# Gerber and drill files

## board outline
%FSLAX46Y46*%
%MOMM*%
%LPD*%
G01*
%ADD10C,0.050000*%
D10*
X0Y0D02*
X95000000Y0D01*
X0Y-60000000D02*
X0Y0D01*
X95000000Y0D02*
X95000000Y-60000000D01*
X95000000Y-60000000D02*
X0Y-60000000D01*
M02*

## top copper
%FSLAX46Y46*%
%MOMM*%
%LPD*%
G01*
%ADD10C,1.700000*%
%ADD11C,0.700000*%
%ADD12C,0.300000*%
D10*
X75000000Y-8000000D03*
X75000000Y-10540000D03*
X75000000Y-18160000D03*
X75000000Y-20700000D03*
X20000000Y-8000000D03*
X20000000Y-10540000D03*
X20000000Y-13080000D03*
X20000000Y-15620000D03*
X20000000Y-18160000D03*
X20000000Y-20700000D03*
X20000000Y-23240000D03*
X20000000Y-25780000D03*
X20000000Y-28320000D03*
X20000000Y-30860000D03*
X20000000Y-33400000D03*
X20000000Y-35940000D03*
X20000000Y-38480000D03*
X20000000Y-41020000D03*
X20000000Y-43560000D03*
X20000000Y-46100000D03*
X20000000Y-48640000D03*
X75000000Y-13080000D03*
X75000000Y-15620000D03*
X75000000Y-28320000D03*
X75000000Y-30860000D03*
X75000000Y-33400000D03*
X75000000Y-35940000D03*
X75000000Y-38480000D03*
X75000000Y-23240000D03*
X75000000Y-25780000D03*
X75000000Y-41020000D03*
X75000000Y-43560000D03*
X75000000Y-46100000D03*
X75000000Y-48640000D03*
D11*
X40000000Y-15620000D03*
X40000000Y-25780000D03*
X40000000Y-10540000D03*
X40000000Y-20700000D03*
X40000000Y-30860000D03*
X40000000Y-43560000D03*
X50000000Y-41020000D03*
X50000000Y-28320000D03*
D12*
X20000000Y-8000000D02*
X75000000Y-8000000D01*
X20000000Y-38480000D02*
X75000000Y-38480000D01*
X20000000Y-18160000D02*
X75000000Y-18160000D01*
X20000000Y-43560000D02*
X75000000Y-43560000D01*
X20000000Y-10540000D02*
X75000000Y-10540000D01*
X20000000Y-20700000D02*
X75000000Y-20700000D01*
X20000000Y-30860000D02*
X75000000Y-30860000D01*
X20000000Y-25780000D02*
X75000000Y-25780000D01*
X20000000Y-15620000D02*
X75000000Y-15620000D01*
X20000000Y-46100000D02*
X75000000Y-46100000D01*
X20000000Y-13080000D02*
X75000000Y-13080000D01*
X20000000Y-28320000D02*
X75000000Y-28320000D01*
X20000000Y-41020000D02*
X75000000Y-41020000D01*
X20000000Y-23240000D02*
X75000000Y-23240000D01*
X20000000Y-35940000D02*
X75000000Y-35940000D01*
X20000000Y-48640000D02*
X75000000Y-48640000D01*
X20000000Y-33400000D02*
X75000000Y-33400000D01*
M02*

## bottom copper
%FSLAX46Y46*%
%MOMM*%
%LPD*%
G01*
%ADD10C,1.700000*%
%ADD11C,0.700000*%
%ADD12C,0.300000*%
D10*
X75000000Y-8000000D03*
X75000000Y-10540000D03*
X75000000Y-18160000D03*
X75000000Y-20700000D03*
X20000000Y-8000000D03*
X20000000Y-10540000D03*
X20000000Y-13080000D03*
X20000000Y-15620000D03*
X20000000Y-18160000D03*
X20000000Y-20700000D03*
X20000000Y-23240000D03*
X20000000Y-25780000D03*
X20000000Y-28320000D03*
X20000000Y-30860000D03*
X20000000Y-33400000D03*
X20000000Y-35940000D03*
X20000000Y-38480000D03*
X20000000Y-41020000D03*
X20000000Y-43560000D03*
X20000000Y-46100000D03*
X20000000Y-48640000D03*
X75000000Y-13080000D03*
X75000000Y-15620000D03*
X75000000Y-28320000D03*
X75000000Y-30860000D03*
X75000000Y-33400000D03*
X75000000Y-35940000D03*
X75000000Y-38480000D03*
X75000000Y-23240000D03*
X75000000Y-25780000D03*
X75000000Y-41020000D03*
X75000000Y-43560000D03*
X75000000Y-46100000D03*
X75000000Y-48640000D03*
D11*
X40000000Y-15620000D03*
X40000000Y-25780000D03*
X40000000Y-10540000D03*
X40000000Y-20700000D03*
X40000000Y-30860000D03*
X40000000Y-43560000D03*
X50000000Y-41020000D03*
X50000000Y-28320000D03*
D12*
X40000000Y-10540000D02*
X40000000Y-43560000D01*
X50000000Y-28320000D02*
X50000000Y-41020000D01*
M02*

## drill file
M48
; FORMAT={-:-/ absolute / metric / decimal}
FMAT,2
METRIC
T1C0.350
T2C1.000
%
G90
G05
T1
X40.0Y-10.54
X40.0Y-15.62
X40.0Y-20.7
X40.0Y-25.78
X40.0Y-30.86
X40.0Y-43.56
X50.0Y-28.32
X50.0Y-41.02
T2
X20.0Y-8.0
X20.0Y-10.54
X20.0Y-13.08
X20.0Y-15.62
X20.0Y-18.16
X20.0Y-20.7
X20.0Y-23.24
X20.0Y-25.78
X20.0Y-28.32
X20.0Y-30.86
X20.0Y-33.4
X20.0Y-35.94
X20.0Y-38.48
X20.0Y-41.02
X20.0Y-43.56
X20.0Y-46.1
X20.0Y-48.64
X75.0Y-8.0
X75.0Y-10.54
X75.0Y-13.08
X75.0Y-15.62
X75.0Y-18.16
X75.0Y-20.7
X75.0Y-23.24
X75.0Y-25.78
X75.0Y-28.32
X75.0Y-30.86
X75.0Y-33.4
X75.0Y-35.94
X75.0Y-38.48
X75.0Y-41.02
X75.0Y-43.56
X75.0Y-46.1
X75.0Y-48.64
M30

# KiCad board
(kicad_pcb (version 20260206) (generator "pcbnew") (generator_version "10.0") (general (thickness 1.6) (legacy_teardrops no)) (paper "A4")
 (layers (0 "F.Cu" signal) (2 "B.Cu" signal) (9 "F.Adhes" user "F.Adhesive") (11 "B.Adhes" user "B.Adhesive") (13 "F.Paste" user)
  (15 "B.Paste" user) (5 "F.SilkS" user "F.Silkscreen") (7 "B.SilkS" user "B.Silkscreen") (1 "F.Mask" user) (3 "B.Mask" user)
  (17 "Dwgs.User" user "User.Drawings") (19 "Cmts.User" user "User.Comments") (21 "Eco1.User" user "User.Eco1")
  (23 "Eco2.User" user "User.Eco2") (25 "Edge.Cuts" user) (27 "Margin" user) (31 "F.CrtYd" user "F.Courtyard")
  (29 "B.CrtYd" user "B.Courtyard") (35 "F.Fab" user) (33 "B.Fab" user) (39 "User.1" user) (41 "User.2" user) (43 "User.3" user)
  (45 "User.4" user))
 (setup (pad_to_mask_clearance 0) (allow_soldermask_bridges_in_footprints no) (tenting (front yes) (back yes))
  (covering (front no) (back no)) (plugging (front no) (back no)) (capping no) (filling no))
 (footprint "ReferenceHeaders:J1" (layer "F.Cu") (at 75 8)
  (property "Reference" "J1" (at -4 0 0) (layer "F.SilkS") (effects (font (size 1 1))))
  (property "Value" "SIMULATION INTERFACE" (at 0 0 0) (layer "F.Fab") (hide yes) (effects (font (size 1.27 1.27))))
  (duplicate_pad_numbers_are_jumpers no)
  (pad "1" thru_hole circle (at 0 0) (size 1.7 1.7) (drill 1) (layers "*.Cu" "*.Mask") (remove_unused_layers no) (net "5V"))
  (pad "2" thru_hole circle (at 0 2.54) (size 1.7 1.7) (drill 1) (layers "*.Cu" "*.Mask") (remove_unused_layers no) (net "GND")))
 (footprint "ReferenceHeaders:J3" (layer "F.Cu") (at 75 18.16)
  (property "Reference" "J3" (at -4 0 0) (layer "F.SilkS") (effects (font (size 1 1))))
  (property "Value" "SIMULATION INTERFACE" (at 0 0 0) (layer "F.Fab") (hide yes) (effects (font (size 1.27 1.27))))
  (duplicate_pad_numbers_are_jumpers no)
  (pad "1" thru_hole circle (at 0 0) (size 1.7 1.7) (drill 1) (layers "*.Cu" "*.Mask") (remove_unused_layers no) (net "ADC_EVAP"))
  (pad "2" thru_hole circle (at 0 2.54) (size 1.7 1.7) (drill 1) (layers "*.Cu" "*.Mask") (remove_unused_layers no) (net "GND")))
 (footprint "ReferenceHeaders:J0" (layer "F.Cu") (at 20 8)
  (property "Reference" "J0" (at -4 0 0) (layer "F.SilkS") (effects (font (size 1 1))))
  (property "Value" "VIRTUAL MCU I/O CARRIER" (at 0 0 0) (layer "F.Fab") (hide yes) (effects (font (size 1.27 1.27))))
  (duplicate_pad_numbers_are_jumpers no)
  (pad "1" thru_hole circle (at 0 0) (size 1.7 1.7) (drill 1) (layers "*.Cu" "*.Mask") (remove_unused_layers no) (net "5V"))
  (pad "2" thru_hole circle (at 0 2.54) (size 1.7 1.7) (drill 1) (layers "*.Cu" "*.Mask") (remove_unused_layers no) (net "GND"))
  (pad "3" thru_hole circle (at 0 5.08) (size 1.7 1.7) (drill 1) (layers "*.Cu" "*.Mask") (remove_unused_layers no) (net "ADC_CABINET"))
  (pad "4" thru_hole circle (at 0 7.62) (size 1.7 1.7) (drill 1) (layers "*.Cu" "*.Mask") (remove_unused_layers no) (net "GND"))
  (pad "5" thru_hole circle (at 0 10.16) (size 1.7 1.7) (drill 1) (layers "*.Cu" "*.Mask") (remove_unused_layers no) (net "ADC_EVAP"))
  (pad "6" thru_hole circle (at 0 12.7) (size 1.7 1.7) (drill 1) (layers "*.Cu" "*.Mask") (remove_unused_layers no) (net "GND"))
  (pad "7" thru_hole circle (at 0 15.24) (size 1.7 1.7) (drill 1) (layers "*.Cu" "*.Mask") (remove_unused_layers no)
   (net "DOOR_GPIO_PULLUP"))
  (pad "8" thru_hole circle (at 0 17.78) (size 1.7 1.7) (drill 1) (layers "*.Cu" "*.Mask") (remove_unused_layers no) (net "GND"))
  (pad "9" thru_hole circle (at 0 20.32) (size 1.7 1.7) (drill 1) (layers "*.Cu" "*.Mask") (remove_unused_layers no) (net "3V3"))
  (pad "10" thru_hole circle (at 0 22.86) (size 1.7 1.7) (drill 1) (layers "*.Cu" "*.Mask") (remove_unused_layers no) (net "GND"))
  (pad "11" thru_hole circle (at 0 25.4) (size 1.7 1.7) (drill 1) (layers "*.Cu" "*.Mask") (remove_unused_layers no) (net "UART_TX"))
  (pad "12" thru_hole circle (at 0 27.94) (size 1.7 1.7) (drill 1) (layers "*.Cu" "*.Mask") (remove_unused_layers no) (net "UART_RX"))
  (pad "13" thru_hole circle (at 0 30.48) (size 1.7 1.7) (drill 1) (layers "*.Cu" "*.Mask") (remove_unused_layers no) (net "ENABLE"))
  (pad "14" thru_hole circle (at 0 33.02) (size 1.7 1.7) (drill 1) (layers "*.Cu" "*.Mask") (remove_unused_layers no) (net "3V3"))
  (pad "15" thru_hole circle (at 0 35.56) (size 1.7 1.7) (drill 1) (layers "*.Cu" "*.Mask") (remove_unused_layers no) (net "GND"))
  (pad "16" thru_hole circle (at 0 38.1) (size 1.7 1.7) (drill 1) (layers "*.Cu" "*.Mask") (remove_unused_layers no) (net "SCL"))
  (pad "17" thru_hole circle (at 0 40.64) (size 1.7 1.7) (drill 1) (layers "*.Cu" "*.Mask") (remove_unused_layers no) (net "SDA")))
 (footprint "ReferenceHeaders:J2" (layer "F.Cu") (at 75 13.08)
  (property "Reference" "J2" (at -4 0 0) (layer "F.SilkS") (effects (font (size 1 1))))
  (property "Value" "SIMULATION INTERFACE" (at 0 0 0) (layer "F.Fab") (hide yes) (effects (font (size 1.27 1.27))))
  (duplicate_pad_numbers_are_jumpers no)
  (pad "1" thru_hole circle (at 0 0) (size 1.7 1.7) (drill 1) (layers "*.Cu" "*.Mask") (remove_unused_layers no) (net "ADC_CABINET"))
  (pad "2" thru_hole circle (at 0 2.54) (size 1.7 1.7) (drill 1) (layers "*.Cu" "*.Mask") (remove_unused_layers no) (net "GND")))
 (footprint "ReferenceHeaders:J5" (layer "F.Cu") (at 75 28.32)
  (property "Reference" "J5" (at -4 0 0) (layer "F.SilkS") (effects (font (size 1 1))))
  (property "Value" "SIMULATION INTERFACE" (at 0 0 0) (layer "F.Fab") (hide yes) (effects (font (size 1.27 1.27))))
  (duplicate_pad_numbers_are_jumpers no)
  (pad "1" thru_hole circle (at 0 0) (size 1.7 1.7) (drill 1) (layers "*.Cu" "*.Mask") (remove_unused_layers no) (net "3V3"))
  (pad "2" thru_hole circle (at 0 2.54) (size 1.7 1.7) (drill 1) (layers "*.Cu" "*.Mask") (remove_unused_layers no) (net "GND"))
  (pad "3" thru_hole circle (at 0 5.08) (size 1.7 1.7) (drill 1) (layers "*.Cu" "*.Mask") (remove_unused_layers no) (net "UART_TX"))
  (pad "4" thru_hole circle (at 0 7.62) (size 1.7 1.7) (drill 1) (layers "*.Cu" "*.Mask") (remove_unused_layers no) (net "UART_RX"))
  (pad "5" thru_hole circle (at 0 10.16) (size 1.7 1.7) (drill 1) (layers "*.Cu" "*.Mask") (remove_unused_layers no) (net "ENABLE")))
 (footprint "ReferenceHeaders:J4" (layer "F.Cu") (at 75 23.24)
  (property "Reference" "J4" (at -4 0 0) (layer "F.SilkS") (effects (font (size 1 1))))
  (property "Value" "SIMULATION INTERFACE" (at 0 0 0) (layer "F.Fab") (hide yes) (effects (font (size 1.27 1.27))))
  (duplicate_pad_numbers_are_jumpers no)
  (pad "1" thru_hole circle (at 0 0) (size 1.7 1.7) (drill 1) (layers "*.Cu" "*.Mask") (remove_unused_layers no) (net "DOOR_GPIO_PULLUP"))
  (pad "2" thru_hole circle (at 0 2.54) (size 1.7 1.7) (drill 1) (layers "*.Cu" "*.Mask") (remove_unused_layers no) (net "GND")))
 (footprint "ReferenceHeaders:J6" (layer "F.Cu") (at 75 41.02)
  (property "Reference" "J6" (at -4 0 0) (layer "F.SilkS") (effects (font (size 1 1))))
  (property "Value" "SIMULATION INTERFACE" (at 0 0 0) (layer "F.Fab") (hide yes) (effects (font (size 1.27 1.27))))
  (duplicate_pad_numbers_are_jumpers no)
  (pad "1" thru_hole circle (at 0 0) (size 1.7 1.7) (drill 1) (layers "*.Cu" "*.Mask") (remove_unused_layers no) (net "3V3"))
  (pad "2" thru_hole circle (at 0 2.54) (size 1.7 1.7) (drill 1) (layers "*.Cu" "*.Mask") (remove_unused_layers no) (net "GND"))
  (pad "3" thru_hole circle (at 0 5.08) (size 1.7 1.7) (drill 1) (layers "*.Cu" "*.Mask") (remove_unused_layers no) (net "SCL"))
  (pad "4" thru_hole circle (at 0 7.62) (size 1.7 1.7) (drill 1) (layers "*.Cu" "*.Mask") (remove_unused_layers no) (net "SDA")))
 (gr_line (start 0 0) (end 95 0) (stroke (width 0.05) (type default)) (layer "Edge.Cuts"))
 (gr_line (start 0 60) (end 0 0) (stroke (width 0.05) (type default)) (layer "Edge.Cuts"))
 (gr_line (start 95 0) (end 95 60) (stroke (width 0.05) (type default)) (layer "Edge.Cuts"))
 (gr_line (start 95 60) (end 0 60) (stroke (width 0.05) (type default)) (layer "Edge.Cuts"))
 (segment (start 20 8) (end 75 8) (width 0.3) (layer "F.Cu") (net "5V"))
 (segment (start 20 38.48) (end 75 38.48) (width 0.3) (layer "F.Cu") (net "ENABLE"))
 (segment (start 20 18.16) (end 75 18.16) (width 0.3) (layer "F.Cu") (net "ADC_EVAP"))
 (segment (start 20 43.56) (end 75 43.56) (width 0.3) (layer "F.Cu") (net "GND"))
 (segment (start 20 10.54) (end 75 10.54) (width 0.3) (layer "F.Cu") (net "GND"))
 (segment (start 20 20.7) (end 75 20.7) (width 0.3) (layer "F.Cu") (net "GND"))
 (segment (start 20 30.86) (end 75 30.86) (width 0.3) (layer "F.Cu") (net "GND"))
 (segment (start 20 25.78) (end 75 25.78) (width 0.3) (layer "F.Cu") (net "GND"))
 (segment (start 20 15.62) (end 75 15.62) (width 0.3) (layer "F.Cu") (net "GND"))
 (via (at 40 15.62) (size 0.7) (drill 0.35) (layers "F.Cu" "B.Cu") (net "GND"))
 (via (at 40 25.78) (size 0.7) (drill 0.35) (layers "F.Cu" "B.Cu") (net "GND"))
 (via (at 40 10.54) (size 0.7) (drill 0.35) (layers "F.Cu" "B.Cu") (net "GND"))
 (via (at 40 20.7) (size 0.7) (drill 0.35) (layers "F.Cu" "B.Cu") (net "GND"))
 (via (at 40 30.86) (size 0.7) (drill 0.35) (layers "F.Cu" "B.Cu") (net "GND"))
 (via (at 40 43.56) (size 0.7) (drill 0.35) (layers "F.Cu" "B.Cu") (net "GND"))
 (segment (start 40 10.54) (end 40 43.56) (width 0.3) (layer "B.Cu") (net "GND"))
 (segment (start 20 46.1) (end 75 46.1) (width 0.3) (layer "F.Cu") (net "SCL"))
 (segment (start 20 13.08) (end 75 13.08) (width 0.3) (layer "F.Cu") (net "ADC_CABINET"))
 (segment (start 20 28.32) (end 75 28.32) (width 0.3) (layer "F.Cu") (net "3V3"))
 (segment (start 20 41.02) (end 75 41.02) (width 0.3) (layer "F.Cu") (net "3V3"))
 (via (at 50 41.02) (size 0.7) (drill 0.35) (layers "F.Cu" "B.Cu") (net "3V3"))
 (via (at 50 28.32) (size 0.7) (drill 0.35) (layers "F.Cu" "B.Cu") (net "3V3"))
 (segment (start 50 28.32) (end 50 41.02) (width 0.3) (layer "B.Cu") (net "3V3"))
 (segment (start 20 23.24) (end 75 23.24) (width 0.3) (layer "F.Cu") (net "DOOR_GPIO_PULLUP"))
 (segment (start 20 35.94) (end 75 35.94) (width 0.3) (layer "F.Cu") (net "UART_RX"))
 (segment (start 20 48.64) (end 75 48.64) (width 0.3) (layer "F.Cu") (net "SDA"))
 (segment (start 20 33.4) (end 75 33.4) (width 0.3) (layer "F.Cu") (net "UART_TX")))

